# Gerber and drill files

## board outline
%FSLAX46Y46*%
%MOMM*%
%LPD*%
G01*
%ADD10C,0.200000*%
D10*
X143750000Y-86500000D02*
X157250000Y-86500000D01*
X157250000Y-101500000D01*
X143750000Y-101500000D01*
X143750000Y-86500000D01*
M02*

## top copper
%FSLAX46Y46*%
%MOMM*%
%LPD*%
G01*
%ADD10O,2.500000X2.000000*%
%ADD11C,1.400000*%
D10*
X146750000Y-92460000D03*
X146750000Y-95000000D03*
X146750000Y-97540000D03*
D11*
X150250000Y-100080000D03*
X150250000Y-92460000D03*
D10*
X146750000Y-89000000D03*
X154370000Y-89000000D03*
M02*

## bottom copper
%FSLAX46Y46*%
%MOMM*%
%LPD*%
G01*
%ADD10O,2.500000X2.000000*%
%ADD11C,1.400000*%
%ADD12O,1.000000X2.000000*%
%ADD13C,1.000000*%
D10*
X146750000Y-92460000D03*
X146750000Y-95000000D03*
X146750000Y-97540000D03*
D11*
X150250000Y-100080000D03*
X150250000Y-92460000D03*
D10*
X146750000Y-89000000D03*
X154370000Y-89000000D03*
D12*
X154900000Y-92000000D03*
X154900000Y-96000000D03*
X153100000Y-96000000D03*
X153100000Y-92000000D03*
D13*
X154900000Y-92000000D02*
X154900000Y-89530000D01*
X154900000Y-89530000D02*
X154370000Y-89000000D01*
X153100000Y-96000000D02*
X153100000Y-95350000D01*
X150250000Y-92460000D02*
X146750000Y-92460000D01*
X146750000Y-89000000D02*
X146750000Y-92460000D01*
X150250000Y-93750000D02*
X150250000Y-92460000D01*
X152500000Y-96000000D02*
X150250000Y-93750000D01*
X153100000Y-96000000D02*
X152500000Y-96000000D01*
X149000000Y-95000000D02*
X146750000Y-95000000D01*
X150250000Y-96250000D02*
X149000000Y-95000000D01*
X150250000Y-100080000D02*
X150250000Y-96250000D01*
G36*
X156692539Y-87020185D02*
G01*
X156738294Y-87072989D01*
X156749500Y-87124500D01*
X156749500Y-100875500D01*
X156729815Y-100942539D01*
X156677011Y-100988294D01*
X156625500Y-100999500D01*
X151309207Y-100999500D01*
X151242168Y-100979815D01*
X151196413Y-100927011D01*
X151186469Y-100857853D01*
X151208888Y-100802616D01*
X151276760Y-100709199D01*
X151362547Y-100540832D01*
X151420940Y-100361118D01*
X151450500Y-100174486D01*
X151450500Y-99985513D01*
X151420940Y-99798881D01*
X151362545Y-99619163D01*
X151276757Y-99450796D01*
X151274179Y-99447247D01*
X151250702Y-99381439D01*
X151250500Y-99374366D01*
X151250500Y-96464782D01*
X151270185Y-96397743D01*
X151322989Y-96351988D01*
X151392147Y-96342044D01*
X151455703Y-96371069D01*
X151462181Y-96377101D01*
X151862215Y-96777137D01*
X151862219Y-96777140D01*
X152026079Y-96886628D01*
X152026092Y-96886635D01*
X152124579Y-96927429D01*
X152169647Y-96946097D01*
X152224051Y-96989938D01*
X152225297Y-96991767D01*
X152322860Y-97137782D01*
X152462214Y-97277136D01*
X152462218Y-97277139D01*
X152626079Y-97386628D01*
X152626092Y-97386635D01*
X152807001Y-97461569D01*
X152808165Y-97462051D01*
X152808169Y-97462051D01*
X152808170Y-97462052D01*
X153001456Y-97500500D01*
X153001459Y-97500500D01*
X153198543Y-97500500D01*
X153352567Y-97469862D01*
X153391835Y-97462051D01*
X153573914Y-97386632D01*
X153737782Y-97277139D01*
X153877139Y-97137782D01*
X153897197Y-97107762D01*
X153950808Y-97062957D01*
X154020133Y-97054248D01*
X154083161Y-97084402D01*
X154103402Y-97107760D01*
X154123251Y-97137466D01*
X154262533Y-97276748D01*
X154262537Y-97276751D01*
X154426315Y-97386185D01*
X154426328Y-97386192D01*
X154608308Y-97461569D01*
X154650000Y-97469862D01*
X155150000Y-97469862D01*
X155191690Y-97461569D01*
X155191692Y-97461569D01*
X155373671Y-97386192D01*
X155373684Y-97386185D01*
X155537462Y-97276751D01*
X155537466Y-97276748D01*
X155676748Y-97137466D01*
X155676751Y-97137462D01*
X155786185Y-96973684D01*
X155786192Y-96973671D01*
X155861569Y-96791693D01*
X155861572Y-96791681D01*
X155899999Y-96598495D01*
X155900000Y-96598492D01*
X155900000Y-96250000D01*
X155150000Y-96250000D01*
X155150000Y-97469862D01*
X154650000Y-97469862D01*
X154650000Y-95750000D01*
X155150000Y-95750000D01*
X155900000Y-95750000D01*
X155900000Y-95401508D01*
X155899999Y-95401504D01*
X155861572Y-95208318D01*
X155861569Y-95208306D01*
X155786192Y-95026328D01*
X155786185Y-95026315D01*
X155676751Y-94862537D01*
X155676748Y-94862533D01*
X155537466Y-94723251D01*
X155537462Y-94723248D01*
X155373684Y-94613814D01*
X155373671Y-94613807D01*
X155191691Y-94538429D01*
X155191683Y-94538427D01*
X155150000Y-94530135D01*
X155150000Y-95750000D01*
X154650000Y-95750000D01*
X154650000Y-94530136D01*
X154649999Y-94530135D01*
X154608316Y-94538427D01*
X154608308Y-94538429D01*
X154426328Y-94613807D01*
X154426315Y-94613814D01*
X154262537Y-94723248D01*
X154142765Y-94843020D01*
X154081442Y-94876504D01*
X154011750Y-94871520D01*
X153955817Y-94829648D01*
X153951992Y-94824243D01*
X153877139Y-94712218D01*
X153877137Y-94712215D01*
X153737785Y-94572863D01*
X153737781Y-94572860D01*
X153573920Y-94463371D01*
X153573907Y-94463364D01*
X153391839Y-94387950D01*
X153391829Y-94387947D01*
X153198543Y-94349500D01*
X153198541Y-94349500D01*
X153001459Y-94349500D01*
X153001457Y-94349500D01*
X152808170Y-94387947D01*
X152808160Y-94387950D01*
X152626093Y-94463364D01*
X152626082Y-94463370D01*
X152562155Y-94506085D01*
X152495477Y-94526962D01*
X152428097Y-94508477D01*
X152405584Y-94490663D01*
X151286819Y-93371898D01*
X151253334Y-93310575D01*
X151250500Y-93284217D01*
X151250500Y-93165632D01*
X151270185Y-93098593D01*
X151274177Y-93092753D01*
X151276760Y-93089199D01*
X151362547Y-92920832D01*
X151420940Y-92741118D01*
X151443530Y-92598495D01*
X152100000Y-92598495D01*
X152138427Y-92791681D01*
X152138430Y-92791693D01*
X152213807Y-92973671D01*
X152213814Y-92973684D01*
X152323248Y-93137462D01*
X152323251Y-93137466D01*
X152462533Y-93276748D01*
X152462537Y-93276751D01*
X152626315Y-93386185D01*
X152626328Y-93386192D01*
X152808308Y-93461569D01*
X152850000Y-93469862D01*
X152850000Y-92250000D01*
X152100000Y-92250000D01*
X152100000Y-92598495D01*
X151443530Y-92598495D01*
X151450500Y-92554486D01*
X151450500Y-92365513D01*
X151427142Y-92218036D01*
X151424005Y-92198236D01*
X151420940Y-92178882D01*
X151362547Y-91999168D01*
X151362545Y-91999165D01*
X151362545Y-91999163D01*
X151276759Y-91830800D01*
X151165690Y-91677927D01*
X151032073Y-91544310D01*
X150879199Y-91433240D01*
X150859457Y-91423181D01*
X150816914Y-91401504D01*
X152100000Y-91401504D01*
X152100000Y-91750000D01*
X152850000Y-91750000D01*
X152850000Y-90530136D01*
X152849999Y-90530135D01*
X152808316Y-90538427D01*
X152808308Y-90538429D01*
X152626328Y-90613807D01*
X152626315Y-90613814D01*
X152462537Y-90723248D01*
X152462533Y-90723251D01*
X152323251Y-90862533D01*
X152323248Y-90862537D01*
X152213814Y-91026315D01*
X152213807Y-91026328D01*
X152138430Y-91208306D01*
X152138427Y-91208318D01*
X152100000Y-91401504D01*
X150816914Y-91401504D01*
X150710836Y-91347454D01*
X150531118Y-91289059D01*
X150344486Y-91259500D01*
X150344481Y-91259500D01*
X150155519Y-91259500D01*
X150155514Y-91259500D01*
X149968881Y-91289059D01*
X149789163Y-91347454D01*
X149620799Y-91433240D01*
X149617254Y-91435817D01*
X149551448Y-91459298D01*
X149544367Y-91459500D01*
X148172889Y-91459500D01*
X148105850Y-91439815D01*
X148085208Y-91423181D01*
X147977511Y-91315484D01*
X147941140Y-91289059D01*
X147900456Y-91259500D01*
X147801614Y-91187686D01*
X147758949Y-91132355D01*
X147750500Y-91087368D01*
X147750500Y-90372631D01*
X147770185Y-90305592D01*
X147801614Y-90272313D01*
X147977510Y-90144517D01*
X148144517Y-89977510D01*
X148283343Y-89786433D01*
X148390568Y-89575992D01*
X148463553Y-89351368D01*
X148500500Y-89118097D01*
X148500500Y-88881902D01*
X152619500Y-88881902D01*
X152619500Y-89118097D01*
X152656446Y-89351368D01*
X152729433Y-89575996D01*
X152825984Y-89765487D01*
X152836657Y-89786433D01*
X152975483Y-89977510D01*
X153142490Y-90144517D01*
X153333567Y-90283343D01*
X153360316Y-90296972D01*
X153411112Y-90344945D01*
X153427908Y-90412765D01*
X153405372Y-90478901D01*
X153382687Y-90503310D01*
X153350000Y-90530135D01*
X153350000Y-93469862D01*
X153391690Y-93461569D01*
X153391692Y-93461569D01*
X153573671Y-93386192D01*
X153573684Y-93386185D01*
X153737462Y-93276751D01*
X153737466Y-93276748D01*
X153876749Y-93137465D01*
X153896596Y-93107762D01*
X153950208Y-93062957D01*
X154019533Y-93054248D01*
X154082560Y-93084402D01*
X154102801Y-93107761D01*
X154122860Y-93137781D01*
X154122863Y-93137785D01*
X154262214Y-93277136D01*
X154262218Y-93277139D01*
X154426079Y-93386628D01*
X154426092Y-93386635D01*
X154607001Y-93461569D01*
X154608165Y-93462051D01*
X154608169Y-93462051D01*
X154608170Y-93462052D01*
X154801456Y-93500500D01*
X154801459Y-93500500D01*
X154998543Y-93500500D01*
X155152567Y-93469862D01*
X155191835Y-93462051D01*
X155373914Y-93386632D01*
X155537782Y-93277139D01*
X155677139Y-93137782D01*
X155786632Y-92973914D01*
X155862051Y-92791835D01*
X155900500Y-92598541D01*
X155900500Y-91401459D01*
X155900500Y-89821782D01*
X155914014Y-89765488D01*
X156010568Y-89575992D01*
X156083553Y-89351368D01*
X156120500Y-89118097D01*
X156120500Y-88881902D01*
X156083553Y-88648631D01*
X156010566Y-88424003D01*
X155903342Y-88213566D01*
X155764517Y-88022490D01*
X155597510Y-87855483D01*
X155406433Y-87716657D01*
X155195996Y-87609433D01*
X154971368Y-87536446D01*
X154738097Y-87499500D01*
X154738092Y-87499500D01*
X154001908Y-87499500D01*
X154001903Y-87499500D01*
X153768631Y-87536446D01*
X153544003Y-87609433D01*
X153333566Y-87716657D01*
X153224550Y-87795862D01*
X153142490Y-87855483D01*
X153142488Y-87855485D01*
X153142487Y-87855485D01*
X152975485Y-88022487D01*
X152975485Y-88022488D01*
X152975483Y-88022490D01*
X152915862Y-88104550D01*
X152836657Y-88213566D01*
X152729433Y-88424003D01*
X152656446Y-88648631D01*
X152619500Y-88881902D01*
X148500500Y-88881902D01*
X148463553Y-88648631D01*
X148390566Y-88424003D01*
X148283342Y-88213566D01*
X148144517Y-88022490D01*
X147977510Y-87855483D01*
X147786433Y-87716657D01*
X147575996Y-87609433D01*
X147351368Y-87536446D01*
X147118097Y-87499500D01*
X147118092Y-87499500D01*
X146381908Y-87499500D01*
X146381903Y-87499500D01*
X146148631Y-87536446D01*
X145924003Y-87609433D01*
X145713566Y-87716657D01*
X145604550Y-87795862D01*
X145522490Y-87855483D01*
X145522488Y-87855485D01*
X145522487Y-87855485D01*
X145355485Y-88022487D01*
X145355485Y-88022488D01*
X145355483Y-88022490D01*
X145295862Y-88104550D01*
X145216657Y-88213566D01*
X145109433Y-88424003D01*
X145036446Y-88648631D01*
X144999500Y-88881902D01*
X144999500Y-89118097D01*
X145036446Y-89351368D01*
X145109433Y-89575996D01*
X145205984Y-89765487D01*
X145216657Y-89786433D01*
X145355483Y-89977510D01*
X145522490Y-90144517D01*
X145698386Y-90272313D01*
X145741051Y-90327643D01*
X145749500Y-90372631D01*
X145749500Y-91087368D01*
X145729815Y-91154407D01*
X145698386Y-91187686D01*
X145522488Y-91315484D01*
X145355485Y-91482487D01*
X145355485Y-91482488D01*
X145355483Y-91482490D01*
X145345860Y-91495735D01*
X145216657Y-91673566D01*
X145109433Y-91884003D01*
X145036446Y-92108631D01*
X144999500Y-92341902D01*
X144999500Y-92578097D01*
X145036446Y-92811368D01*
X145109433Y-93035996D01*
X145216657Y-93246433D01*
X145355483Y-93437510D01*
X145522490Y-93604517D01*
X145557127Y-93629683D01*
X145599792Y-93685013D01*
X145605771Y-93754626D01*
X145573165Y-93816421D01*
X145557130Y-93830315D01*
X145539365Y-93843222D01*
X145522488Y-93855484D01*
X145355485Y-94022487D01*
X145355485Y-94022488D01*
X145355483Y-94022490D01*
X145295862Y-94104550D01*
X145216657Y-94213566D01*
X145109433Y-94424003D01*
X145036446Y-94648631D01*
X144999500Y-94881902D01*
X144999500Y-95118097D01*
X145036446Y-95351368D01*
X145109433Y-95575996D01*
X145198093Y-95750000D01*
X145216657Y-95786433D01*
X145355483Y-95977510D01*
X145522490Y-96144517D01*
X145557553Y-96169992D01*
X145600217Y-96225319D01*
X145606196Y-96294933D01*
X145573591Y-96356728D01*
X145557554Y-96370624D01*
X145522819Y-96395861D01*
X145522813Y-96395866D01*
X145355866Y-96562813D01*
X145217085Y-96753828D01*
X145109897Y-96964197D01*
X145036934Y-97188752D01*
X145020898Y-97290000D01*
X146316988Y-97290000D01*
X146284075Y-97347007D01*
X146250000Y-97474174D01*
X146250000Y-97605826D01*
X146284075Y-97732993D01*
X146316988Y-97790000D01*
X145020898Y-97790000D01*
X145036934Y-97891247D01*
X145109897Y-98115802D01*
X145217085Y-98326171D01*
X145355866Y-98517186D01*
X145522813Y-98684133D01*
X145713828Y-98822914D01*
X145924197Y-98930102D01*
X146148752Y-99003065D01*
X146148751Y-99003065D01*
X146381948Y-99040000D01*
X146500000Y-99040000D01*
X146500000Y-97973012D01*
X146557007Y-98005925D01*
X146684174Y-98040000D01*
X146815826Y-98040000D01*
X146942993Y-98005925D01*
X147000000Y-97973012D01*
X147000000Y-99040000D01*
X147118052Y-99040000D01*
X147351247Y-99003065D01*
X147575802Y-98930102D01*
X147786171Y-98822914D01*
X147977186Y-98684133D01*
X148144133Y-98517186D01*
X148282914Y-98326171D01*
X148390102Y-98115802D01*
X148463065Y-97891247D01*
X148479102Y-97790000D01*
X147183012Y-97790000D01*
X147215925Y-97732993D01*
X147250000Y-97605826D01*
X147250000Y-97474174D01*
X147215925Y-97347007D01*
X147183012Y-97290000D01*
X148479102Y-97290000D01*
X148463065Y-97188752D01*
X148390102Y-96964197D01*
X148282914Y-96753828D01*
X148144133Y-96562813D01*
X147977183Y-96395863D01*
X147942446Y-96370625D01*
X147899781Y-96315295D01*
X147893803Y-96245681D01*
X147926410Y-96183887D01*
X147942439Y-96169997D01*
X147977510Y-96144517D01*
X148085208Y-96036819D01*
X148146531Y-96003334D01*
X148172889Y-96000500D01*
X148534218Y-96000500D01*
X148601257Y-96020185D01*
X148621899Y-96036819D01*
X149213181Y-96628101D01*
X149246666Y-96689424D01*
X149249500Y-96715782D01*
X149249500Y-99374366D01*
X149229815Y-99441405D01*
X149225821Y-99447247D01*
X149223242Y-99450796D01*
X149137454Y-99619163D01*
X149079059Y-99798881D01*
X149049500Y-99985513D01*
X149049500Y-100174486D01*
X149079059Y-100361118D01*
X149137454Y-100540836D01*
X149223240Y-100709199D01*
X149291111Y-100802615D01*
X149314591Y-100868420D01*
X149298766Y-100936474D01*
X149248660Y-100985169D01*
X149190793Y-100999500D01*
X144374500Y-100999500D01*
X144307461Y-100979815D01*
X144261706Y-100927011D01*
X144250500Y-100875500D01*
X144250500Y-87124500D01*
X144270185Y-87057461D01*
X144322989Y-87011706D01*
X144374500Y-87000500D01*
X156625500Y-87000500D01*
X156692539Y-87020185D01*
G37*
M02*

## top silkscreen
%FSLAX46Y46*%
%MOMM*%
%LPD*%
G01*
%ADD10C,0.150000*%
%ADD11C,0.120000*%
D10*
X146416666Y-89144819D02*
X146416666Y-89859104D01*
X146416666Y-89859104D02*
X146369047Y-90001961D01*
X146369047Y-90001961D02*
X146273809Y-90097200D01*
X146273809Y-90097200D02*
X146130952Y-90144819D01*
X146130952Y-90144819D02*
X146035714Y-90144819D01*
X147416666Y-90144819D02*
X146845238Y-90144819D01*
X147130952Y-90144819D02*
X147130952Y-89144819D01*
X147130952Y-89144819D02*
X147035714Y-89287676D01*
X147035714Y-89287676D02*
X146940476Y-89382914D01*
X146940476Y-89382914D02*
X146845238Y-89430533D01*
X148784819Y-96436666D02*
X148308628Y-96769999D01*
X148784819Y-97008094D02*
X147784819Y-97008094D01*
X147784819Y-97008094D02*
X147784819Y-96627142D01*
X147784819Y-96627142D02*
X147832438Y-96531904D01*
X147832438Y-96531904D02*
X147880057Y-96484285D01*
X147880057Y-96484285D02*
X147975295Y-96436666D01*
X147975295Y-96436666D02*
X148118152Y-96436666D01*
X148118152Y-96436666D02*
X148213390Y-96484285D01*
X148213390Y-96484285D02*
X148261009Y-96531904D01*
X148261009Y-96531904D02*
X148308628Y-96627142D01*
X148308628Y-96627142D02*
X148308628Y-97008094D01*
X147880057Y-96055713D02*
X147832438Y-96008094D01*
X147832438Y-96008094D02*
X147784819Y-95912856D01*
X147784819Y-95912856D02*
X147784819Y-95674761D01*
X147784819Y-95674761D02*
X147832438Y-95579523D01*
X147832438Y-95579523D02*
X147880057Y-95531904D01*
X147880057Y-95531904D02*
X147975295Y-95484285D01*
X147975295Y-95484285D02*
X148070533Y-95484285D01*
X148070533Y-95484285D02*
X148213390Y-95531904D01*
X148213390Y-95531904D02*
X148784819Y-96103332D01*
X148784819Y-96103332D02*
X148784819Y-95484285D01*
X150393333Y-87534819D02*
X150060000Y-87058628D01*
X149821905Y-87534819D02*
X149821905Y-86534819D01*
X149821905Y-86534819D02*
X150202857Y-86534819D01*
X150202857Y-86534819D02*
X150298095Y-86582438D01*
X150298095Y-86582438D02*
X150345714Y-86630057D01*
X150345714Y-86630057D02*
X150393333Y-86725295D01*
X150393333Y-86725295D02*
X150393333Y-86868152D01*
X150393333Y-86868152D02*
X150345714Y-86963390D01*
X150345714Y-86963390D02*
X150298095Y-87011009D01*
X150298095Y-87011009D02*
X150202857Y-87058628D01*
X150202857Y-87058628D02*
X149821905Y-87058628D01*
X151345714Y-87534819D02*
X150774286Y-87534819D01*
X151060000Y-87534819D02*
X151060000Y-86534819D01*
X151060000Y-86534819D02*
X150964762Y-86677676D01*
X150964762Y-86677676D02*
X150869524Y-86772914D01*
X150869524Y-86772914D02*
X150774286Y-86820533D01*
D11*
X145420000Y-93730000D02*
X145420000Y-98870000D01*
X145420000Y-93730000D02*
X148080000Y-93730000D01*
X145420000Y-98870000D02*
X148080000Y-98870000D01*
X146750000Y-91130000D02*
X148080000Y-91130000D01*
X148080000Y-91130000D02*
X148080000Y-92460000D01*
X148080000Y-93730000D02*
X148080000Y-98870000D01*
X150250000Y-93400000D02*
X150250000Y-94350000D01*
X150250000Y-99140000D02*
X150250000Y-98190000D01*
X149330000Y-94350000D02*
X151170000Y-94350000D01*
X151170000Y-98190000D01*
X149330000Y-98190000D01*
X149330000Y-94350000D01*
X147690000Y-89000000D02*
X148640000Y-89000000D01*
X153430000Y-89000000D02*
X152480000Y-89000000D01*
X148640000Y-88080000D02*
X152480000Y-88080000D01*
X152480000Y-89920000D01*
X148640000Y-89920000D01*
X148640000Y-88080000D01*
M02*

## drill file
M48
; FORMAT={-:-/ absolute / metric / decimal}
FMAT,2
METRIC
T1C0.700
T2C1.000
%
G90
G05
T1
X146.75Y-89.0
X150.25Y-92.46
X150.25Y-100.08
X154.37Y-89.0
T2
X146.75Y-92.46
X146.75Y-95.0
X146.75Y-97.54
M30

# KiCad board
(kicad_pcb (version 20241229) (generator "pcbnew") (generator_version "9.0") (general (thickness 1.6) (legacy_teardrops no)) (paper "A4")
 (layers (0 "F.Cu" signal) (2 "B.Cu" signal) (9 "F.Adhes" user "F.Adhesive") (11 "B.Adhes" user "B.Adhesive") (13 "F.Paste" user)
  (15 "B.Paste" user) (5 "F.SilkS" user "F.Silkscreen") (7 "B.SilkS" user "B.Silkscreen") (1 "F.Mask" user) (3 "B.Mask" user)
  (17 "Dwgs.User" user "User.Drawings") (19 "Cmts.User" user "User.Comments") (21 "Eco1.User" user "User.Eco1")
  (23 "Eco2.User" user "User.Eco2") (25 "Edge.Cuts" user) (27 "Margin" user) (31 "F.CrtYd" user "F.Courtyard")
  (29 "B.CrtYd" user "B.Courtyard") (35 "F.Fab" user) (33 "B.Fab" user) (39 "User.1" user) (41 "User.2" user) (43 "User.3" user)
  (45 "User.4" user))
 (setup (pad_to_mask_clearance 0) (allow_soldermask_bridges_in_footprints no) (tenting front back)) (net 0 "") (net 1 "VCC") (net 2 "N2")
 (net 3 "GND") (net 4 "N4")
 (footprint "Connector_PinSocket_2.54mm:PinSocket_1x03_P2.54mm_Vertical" (layer "F.Cu") (at 146.75 92.46)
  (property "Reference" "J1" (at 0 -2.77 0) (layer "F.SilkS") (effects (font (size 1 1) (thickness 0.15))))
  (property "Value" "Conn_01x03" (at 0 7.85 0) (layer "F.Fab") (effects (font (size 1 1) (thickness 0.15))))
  (fp_line (start -1.33 1.27) (end -1.33 6.41) (stroke (width 0.12) (type solid)) (layer "F.SilkS"))
  (fp_line (start -1.33 1.27) (end 1.33 1.27) (stroke (width 0.12) (type solid)) (layer "F.SilkS"))
  (fp_line (start -1.33 6.41) (end 1.33 6.41) (stroke (width 0.12) (type solid)) (layer "F.SilkS"))
  (fp_line (start 0 -1.33) (end 1.33 -1.33) (stroke (width 0.12) (type solid)) (layer "F.SilkS"))
  (fp_line (start 1.33 -1.33) (end 1.33 0) (stroke (width 0.12) (type solid)) (layer "F.SilkS"))
  (fp_line (start 1.33 1.27) (end 1.33 6.41) (stroke (width 0.12) (type solid)) (layer "F.SilkS"))
  (pad "1" thru_hole oval (at 0 0) (size 2.5 2) (drill 1) (layers "*.Cu" "*.Mask") (remove_unused_layers no) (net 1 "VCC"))
  (pad "2" thru_hole oval (at 0 2.54) (size 2.5 2) (drill 1) (layers "*.Cu" "*.Mask") (remove_unused_layers no) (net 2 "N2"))
  (pad "3" thru_hole oval (at 0 5.08) (size 2.5 2) (drill 1) (layers "*.Cu" "*.Mask") (remove_unused_layers no) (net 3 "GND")))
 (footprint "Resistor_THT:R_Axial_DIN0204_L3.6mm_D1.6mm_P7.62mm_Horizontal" (layer "F.Cu") (at 150.25 100.08 90)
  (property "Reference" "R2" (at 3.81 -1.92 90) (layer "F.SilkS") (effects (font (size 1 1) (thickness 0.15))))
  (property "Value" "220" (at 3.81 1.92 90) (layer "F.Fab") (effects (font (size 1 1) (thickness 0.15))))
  (fp_line (start 6.68 0) (end 5.73 0) (stroke (width 0.12) (type solid)) (layer "F.SilkS"))
  (fp_line (start 0.94 0) (end 1.89 0) (stroke (width 0.12) (type solid)) (layer "F.SilkS"))
  (fp_rect (start 1.89 -0.92) (end 5.73 0.92) (stroke (width 0.12) (type solid)) (fill no) (layer "F.SilkS"))
  (pad "1" thru_hole circle (at 0 0 90) (size 1.4 1.4) (drill 0.7) (layers "*.Cu" "*.Mask") (remove_unused_layers no) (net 2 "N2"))
  (pad "2" thru_hole circle (at 7.62 0 90) (size 1.4 1.4) (drill 0.7) (layers "*.Cu" "*.Mask") (remove_unused_layers no) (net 1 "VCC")))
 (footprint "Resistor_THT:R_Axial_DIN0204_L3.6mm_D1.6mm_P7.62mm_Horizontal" (layer "F.Cu") (at 146.75 89)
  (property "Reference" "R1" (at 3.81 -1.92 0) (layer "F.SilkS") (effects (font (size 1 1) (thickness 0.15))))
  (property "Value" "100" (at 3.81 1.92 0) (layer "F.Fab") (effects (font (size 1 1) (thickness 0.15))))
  (fp_line (start 0.94 0) (end 1.89 0) (stroke (width 0.12) (type solid)) (layer "F.SilkS"))
  (fp_line (start 6.68 0) (end 5.73 0) (stroke (width 0.12) (type solid)) (layer "F.SilkS"))
  (fp_rect (start 1.89 -0.92) (end 5.73 0.92) (stroke (width 0.12) (type solid)) (fill no) (layer "F.SilkS"))
  (pad "1" thru_hole oval (at 0 0) (size 2.5 2) (drill 0.7) (layers "*.Cu" "*.Mask") (remove_unused_layers no) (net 1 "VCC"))
  (pad "2" thru_hole oval (at 7.62 0) (size 2.5 2) (drill 0.7) (layers "*.Cu" "*.Mask") (remove_unused_layers no) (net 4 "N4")))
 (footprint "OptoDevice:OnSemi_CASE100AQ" (layer "B.Cu") (at 154.9 92 180)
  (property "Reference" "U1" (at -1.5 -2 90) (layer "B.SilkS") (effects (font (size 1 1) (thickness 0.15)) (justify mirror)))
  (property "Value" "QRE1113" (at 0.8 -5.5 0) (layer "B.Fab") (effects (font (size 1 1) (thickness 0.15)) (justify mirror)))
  (pad "1" smd oval (at 0 0 180) (size 1 2) (layers "B.Cu" "B.Mask" "B.Paste") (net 4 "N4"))
  (pad "2" smd oval (at 0 -4 180) (size 1 2) (layers "B.Cu" "B.Mask" "B.Paste") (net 3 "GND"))
  (pad "3" smd oval (at 1.8 -4 180) (size 1 2) (layers "B.Cu" "B.Mask" "B.Paste") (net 1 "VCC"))
  (pad "4" smd oval (at 1.8 0 180) (size 1 2) (layers "B.Cu" "B.Mask" "B.Paste") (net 3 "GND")))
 (gr_rect (start 143.75 86.5) (end 157.25 101.5) (stroke (width 0.2) (type solid)) (fill no) (layer "Edge.Cuts"))
 (segment (start 154.9 92) (end 154.9 89.53) (width 1) (layer "B.Cu") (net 4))
 (segment (start 154.9 89.53) (end 154.37 89) (width 1) (layer "B.Cu") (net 4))
 (segment (start 153.1 96) (end 153.1 95.35) (width 1) (layer "B.Cu") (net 1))
 (segment (start 150.25 92.46) (end 146.75 92.46) (width 1) (layer "B.Cu") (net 1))
 (segment (start 146.75 89) (end 146.75 92.46) (width 1) (layer "B.Cu") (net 1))
 (segment (start 150.25 93.75) (end 150.25 92.46) (width 1) (layer "B.Cu") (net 1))
 (segment (start 152.5 96) (end 150.25 93.75) (width 1) (layer "B.Cu") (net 1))
 (segment (start 153.1 96) (end 152.5 96) (width 1) (layer "B.Cu") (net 1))
 (segment (start 149 95) (end 146.75 95) (width 1) (layer "B.Cu") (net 2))
 (segment (start 150.25 96.25) (end 149 95) (width 1) (layer "B.Cu") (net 2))
 (segment (start 150.25 100.08) (end 150.25 96.25) (width 1) (layer "B.Cu") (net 2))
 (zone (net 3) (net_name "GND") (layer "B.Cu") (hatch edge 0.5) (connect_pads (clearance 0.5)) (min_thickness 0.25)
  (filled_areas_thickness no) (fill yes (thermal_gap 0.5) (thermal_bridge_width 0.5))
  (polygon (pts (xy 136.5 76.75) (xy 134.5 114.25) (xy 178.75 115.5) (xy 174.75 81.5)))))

